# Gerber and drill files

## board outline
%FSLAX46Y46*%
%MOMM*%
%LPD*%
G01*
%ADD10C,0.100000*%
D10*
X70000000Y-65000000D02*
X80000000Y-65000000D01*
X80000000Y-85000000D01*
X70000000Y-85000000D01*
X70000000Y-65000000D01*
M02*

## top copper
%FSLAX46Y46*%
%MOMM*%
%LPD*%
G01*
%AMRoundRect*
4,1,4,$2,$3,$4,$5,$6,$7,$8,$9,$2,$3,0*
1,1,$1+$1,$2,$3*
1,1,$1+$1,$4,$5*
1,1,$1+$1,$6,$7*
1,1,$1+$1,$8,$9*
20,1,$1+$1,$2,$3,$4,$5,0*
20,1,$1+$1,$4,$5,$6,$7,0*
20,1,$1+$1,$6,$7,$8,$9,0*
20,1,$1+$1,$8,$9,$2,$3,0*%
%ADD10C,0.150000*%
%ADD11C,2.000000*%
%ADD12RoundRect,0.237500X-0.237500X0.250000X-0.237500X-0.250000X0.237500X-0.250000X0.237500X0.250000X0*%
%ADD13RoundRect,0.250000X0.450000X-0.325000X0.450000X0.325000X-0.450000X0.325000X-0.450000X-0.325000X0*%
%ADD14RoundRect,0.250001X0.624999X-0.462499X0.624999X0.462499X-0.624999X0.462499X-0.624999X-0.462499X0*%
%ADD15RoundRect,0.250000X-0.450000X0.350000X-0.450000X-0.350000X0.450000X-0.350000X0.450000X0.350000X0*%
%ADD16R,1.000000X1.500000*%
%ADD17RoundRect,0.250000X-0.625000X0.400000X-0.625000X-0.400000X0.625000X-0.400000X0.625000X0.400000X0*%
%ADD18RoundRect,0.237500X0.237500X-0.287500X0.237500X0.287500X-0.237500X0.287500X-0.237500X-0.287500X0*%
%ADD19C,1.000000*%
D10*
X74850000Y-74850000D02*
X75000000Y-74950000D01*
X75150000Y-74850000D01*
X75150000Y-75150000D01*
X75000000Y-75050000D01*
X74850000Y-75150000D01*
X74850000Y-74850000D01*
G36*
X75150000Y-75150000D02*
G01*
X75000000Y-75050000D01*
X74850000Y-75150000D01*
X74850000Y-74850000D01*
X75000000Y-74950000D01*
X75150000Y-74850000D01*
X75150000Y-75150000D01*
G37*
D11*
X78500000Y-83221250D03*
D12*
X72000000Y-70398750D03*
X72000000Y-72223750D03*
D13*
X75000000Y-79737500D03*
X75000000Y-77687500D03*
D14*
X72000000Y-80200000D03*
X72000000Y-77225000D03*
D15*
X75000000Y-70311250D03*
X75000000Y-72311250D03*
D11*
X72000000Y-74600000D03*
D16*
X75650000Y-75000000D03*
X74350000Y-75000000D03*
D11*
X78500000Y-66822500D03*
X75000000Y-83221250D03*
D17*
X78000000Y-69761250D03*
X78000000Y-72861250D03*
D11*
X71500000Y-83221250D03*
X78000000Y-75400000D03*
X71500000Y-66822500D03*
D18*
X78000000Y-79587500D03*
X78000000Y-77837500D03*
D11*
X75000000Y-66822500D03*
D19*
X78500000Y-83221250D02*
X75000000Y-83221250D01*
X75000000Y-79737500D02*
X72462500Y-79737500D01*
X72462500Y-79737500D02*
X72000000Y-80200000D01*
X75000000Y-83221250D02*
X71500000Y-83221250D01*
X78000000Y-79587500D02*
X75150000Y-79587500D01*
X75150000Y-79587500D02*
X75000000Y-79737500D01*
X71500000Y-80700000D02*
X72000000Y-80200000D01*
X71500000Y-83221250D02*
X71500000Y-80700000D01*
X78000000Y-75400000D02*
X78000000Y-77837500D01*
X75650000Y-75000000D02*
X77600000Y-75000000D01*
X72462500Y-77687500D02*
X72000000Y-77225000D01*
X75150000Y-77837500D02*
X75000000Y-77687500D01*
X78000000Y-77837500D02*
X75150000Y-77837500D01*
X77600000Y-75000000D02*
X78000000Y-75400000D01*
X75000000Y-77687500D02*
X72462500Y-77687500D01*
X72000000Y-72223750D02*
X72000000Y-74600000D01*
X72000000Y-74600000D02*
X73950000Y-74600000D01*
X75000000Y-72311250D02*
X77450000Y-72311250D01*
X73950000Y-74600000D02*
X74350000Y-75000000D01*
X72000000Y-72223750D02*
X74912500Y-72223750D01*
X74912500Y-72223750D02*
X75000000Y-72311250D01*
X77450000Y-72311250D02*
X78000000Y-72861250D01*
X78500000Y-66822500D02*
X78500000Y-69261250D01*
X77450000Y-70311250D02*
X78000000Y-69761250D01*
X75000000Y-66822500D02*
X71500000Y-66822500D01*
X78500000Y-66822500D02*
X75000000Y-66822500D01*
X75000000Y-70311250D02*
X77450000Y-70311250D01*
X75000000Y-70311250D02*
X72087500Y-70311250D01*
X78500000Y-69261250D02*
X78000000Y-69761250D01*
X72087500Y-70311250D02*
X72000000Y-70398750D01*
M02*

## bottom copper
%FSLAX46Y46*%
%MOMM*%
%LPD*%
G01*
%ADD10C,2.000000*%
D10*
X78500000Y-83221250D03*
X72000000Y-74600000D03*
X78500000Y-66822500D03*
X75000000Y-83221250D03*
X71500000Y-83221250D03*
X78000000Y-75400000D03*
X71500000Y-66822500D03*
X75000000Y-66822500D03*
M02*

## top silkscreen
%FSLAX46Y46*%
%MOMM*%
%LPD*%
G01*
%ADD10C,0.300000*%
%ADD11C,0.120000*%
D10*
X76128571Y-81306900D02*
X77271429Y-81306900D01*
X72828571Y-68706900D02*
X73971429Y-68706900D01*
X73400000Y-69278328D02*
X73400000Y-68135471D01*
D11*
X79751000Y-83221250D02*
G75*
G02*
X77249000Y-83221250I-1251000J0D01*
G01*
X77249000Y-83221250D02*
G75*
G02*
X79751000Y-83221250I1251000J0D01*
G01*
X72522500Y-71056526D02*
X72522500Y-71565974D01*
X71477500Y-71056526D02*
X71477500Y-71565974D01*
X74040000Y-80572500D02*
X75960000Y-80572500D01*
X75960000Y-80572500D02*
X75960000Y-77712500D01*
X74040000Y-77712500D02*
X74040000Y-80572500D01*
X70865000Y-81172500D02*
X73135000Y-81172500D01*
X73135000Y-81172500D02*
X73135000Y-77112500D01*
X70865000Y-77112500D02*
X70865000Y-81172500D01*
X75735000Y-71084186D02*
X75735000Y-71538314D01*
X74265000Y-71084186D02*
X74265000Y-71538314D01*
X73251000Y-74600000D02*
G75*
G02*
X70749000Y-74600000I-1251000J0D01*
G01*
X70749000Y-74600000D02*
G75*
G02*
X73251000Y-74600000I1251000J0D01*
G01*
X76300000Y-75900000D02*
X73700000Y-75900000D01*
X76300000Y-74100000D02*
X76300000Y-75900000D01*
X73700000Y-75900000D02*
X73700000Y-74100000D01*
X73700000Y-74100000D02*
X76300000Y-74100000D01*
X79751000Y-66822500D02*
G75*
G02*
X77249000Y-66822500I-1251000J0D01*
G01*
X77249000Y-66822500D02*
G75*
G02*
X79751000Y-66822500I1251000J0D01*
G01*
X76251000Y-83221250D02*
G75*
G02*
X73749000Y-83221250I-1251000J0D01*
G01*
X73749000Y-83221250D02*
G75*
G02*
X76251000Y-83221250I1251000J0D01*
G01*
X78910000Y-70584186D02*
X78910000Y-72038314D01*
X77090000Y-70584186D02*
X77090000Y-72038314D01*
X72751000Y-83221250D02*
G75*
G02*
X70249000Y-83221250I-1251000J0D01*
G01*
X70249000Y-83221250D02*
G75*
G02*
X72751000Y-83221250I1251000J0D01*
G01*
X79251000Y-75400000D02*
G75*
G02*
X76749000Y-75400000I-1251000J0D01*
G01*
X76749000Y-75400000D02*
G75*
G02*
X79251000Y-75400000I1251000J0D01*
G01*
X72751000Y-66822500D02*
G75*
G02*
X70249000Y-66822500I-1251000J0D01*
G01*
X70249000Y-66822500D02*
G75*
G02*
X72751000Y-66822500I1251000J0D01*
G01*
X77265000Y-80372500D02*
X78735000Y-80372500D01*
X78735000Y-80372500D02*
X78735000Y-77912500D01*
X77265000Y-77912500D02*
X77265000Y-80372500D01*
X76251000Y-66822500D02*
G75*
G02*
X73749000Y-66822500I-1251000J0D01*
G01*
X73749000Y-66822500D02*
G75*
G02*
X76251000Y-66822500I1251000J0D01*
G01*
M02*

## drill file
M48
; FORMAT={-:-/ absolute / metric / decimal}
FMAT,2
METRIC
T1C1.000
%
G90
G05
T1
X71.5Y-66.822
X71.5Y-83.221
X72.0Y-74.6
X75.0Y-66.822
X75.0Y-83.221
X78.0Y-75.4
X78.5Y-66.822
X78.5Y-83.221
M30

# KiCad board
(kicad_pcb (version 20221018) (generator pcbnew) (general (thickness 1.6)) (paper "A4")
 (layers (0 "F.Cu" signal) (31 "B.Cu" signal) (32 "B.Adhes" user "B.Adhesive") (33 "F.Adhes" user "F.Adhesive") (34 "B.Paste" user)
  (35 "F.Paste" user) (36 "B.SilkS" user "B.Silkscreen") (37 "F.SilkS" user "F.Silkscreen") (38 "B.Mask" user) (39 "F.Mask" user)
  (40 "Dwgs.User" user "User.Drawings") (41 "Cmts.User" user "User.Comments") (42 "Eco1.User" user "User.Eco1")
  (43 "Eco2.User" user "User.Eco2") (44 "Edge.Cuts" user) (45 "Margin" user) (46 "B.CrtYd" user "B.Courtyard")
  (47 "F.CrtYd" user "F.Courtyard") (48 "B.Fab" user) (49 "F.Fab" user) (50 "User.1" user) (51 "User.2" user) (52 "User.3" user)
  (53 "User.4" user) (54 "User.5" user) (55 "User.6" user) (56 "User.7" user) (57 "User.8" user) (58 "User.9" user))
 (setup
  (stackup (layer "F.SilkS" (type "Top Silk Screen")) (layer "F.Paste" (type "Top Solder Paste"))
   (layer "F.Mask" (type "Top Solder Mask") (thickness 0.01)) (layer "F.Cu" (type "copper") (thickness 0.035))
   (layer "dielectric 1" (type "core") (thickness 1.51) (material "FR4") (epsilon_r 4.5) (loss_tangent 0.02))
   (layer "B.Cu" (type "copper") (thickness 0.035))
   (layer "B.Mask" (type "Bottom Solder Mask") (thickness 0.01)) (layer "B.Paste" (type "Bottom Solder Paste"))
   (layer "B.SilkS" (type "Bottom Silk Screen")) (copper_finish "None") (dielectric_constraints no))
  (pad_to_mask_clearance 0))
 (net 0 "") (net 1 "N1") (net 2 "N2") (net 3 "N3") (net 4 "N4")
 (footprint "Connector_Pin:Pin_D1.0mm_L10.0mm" (layer "F.Cu") (at 78.5 83.22125)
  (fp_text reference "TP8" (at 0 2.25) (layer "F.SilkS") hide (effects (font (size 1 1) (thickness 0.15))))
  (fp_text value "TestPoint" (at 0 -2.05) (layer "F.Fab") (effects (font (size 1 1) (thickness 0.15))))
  (fp_circle (center 0 0) (end 1.25 0.05) (stroke (width 0.12) (type solid)) (fill none) (layer "F.SilkS"))
  (pad "1" thru_hole circle (at 0 0) (size 2 2) (drill 1) (layers "*.Cu" "*.Mask") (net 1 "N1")))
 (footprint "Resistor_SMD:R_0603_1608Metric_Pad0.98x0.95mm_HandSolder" (layer "F.Cu") (at 72 71.31125 -90)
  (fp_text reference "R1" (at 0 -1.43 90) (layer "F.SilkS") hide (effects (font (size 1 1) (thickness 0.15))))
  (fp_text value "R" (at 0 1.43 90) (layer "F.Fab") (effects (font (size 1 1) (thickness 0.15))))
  (fp_line (start -0.254724 -0.5225) (end 0.254724 -0.5225) (stroke (width 0.12) (type solid)) (layer "F.SilkS"))
  (fp_line (start -0.254724 0.5225) (end 0.254724 0.5225) (stroke (width 0.12) (type solid)) (layer "F.SilkS"))
  (pad "1" smd roundrect (at -0.9125 0 270) (size 0.975 0.95) (layers "F.Cu" "F.Paste" "F.Mask") (roundrect_rratio 0.25) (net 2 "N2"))
  (pad "2" smd roundrect (at 0.9125 0 270) (size 0.975 0.95) (layers "F.Cu" "F.Paste" "F.Mask") (roundrect_rratio 0.25) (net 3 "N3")))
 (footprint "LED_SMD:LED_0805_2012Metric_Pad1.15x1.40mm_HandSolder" (layer "F.Cu") (at 75 78.7125 90)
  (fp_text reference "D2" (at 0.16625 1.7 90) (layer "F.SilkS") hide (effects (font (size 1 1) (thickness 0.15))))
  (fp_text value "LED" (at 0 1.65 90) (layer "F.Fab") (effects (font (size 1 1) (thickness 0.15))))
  (fp_line (start -1.86 -0.96) (end -1.86 0.96) (stroke (width 0.12) (type solid)) (layer "F.SilkS"))
  (fp_line (start -1.86 0.96) (end 1 0.96) (stroke (width 0.12) (type solid)) (layer "F.SilkS"))
  (fp_line (start 1 -0.96) (end -1.86 -0.96) (stroke (width 0.12) (type solid)) (layer "F.SilkS"))
  (pad "1" smd roundrect (at -1.025 0 90) (size 1.15 1.4) (layers "F.Cu" "F.Paste" "F.Mask") (roundrect_rratio 0.2173913043) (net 1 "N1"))
  (pad "2" smd roundrect (at 1.025 0 90) (size 1.15 1.4) (layers "F.Cu" "F.Paste" "F.Mask") (roundrect_rratio 0.2173913043) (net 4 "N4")))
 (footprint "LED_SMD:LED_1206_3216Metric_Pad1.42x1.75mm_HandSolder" (layer "F.Cu") (at 72 78.7125 90)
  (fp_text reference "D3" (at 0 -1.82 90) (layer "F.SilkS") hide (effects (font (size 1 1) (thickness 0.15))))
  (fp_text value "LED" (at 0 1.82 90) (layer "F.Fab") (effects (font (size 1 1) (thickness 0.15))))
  (fp_line (start -2.46 -1.135) (end -2.46 1.135) (stroke (width 0.12) (type solid)) (layer "F.SilkS"))
  (fp_line (start -2.46 1.135) (end 1.6 1.135) (stroke (width 0.12) (type solid)) (layer "F.SilkS"))
  (fp_line (start 1.6 -1.135) (end -2.46 -1.135) (stroke (width 0.12) (type solid)) (layer "F.SilkS"))
  (pad "1" smd roundrect (at -1.4875 0 90) (size 1.425 1.75) (layers "F.Cu" "F.Paste" "F.Mask") (roundrect_rratio 0.1754392982) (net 1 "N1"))
  (pad "2" smd roundrect (at 1.4875 0 90) (size 1.425 1.75) (layers "F.Cu" "F.Paste" "F.Mask") (roundrect_rratio 0.1754392982) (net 4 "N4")))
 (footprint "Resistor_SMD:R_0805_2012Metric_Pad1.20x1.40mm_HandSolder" (layer "F.Cu") (at 75 71.31125 -90)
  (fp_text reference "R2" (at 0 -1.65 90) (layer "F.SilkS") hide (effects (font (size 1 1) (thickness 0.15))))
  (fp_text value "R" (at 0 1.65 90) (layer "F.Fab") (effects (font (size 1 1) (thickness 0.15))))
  (fp_line (start -0.227064 -0.735) (end 0.227064 -0.735) (stroke (width 0.12) (type solid)) (layer "F.SilkS"))
  (fp_line (start -0.227064 0.735) (end 0.227064 0.735) (stroke (width 0.12) (type solid)) (layer "F.SilkS"))
  (pad "1" smd roundrect (at -1 0 270) (size 1.2 1.4) (layers "F.Cu" "F.Paste" "F.Mask") (roundrect_rratio 0.2083333333) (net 2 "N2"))
  (pad "2" smd roundrect (at 1 0 270) (size 1.2 1.4) (layers "F.Cu" "F.Paste" "F.Mask") (roundrect_rratio 0.2083333333) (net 3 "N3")))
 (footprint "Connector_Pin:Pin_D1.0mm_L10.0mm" (layer "F.Cu") (at 72 74.6)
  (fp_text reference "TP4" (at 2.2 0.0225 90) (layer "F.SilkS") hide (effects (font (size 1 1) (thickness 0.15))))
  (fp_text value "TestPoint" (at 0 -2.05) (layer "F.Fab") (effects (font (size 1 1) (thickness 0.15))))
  (fp_circle (center 0 0) (end 1.25 0.05) (stroke (width 0.12) (type solid)) (fill none) (layer "F.SilkS"))
  (pad "1" thru_hole circle (at 0 0) (size 2 2) (drill 1) (layers "*.Cu" "*.Mask") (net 3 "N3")))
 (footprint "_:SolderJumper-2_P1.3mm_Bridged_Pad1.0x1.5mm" (layer "F.Cu") (at 75 75 180) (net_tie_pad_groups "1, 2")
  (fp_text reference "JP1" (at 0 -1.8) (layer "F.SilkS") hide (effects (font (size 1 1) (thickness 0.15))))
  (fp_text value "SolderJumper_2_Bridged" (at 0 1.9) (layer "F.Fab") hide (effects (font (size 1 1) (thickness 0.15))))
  (fp_poly
   (pts (xy 0.15 0.15) (xy 0 0.05) (xy -0.15 0.15) (xy -0.15 -0.15) (xy 0 -0.05) (xy 0.15 -0.15)) (stroke (width 0.15) (type solid))
   (fill solid) (layer "F.Cu"))
  (fp_line (start -1.3 -0.9) (end 1.3 -0.9) (stroke (width 0.12) (type solid)) (layer "F.SilkS"))
  (fp_line (start -1.3 0.9) (end -1.3 -0.9) (stroke (width 0.12) (type solid)) (layer "F.SilkS"))
  (fp_line (start 1.3 -0.9) (end 1.3 0.9) (stroke (width 0.12) (type solid)) (layer "F.SilkS"))
  (fp_line (start 1.3 0.9) (end -1.3 0.9) (stroke (width 0.12) (type solid)) (layer "F.SilkS"))
  (pad "1" smd rect (at -0.65 0 180) (size 1 1.5) (layers "F.Cu" "F.Mask") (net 4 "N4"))
  (pad "2" smd rect (at 0.65 0 180) (size 1 1.5) (layers "F.Cu" "F.Mask") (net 3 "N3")))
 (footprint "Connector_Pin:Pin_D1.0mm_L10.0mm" (layer "F.Cu") (at 78.5 66.8225)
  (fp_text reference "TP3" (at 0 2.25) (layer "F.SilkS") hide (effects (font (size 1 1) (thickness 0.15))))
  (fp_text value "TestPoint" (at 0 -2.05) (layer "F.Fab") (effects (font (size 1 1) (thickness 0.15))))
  (fp_circle (center 0 0) (end 1.25 0.05) (stroke (width 0.12) (type solid)) (fill none) (layer "F.SilkS"))
  (pad "1" thru_hole circle (at 0 0) (size 2 2) (drill 1) (layers "*.Cu" "*.Mask") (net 2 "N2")))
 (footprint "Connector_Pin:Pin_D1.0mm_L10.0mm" (layer "F.Cu") (at 75 83.22125)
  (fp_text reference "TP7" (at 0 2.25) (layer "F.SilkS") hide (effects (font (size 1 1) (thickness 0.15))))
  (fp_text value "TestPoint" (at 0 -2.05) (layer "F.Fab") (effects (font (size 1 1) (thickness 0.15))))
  (fp_circle (center 0 0) (end 1.25 0.05) (stroke (width 0.12) (type solid)) (fill none) (layer "F.SilkS"))
  (pad "1" thru_hole circle (at 0 0) (size 2 2) (drill 1) (layers "*.Cu" "*.Mask") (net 1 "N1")))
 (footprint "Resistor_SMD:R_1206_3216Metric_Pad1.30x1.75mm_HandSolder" (layer "F.Cu") (at 78 71.31125 -90)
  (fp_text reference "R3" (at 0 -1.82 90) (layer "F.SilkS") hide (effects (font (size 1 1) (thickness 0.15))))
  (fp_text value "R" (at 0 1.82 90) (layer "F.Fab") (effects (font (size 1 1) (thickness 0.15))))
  (fp_line (start -0.727064 -0.91) (end 0.727064 -0.91) (stroke (width 0.12) (type solid)) (layer "F.SilkS"))
  (fp_line (start -0.727064 0.91) (end 0.727064 0.91) (stroke (width 0.12) (type solid)) (layer "F.SilkS"))
  (pad "1" smd roundrect (at -1.55 0 270) (size 1.3 1.75) (layers "F.Cu" "F.Paste" "F.Mask") (roundrect_rratio 0.1923076923) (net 2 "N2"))
  (pad "2" smd roundrect (at 1.55 0 270) (size 1.3 1.75) (layers "F.Cu" "F.Paste" "F.Mask") (roundrect_rratio 0.1923076923) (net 3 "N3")))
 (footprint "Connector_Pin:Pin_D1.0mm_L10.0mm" (layer "F.Cu") (at 71.5 83.22125)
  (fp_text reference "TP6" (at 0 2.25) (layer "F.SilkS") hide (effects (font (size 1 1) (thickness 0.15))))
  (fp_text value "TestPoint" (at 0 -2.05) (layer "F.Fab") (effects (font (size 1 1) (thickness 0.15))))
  (fp_circle (center 0 0) (end 1.25 0.05) (stroke (width 0.12) (type solid)) (fill none) (layer "F.SilkS"))
  (pad "1" thru_hole circle (at 0 0) (size 2 2) (drill 1) (layers "*.Cu" "*.Mask") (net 1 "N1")))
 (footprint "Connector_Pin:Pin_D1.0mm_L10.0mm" (layer "F.Cu") (at 78 75.4)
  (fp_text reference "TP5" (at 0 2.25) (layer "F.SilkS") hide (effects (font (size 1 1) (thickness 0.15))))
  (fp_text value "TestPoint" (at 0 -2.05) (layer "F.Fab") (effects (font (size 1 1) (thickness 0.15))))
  (fp_circle (center 0 0) (end 1.25 0.05) (stroke (width 0.12) (type solid)) (fill none) (layer "F.SilkS"))
  (pad "1" thru_hole circle (at 0 0) (size 2 2) (drill 1) (layers "*.Cu" "*.Mask") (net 4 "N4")))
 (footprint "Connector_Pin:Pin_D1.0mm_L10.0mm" (layer "F.Cu") (at 71.5 66.8225)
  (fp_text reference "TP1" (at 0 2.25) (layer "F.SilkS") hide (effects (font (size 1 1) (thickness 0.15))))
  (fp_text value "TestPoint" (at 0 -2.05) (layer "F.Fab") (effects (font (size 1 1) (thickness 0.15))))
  (fp_circle (center 0 0) (end 1.25 0.05) (stroke (width 0.12) (type solid)) (fill none) (layer "F.SilkS"))
  (pad "1" thru_hole circle (at 0 0) (size 2 2) (drill 1) (layers "*.Cu" "*.Mask") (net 2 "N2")))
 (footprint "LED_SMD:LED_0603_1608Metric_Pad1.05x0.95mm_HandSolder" (layer "F.Cu") (at 78 78.7125 90)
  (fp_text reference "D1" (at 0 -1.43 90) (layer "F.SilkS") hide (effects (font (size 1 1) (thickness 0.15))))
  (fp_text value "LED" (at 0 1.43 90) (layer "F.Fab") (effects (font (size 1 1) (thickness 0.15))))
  (fp_line (start -1.66 -0.735) (end -1.66 0.735) (stroke (width 0.12) (type solid)) (layer "F.SilkS"))
  (fp_line (start -1.66 0.735) (end 0.8 0.735) (stroke (width 0.12) (type solid)) (layer "F.SilkS"))
  (fp_line (start 0.8 -0.735) (end -1.66 -0.735) (stroke (width 0.12) (type solid)) (layer "F.SilkS"))
  (pad "1" smd roundrect (at -0.875 0 90) (size 1.05 0.95) (layers "F.Cu" "F.Paste" "F.Mask") (roundrect_rratio 0.25) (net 1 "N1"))
  (pad "2" smd roundrect (at 0.875 0 90) (size 1.05 0.95) (layers "F.Cu" "F.Paste" "F.Mask") (roundrect_rratio 0.25) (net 4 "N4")))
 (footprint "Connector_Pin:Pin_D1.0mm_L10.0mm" (layer "F.Cu") (at 75 66.8225)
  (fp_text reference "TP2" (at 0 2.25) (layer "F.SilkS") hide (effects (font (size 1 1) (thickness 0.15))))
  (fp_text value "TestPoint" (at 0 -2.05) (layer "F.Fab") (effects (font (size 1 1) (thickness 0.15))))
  (fp_circle (center 0 0) (end 1.25 0.05) (stroke (width 0.12) (type solid)) (fill none) (layer "F.SilkS"))
  (pad "1" thru_hole circle (at 0 0) (size 2 2) (drill 1) (layers "*.Cu" "*.Mask") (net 2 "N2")))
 (gr_rect (start 70 65) (end 80 85) (stroke (width 0.1) (type solid)) (fill none) (layer "Edge.Cuts"))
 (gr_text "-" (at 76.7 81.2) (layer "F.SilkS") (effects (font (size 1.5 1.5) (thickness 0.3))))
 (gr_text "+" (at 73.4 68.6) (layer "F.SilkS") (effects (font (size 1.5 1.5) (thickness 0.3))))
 (segment (start 78.5 83.22125) (end 75 83.22125) (width 1) (layer "F.Cu") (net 1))
 (segment (start 75 79.7375) (end 72.4625 79.7375) (width 1) (layer "F.Cu") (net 1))
 (segment (start 72.4625 79.7375) (end 72 80.2) (width 1) (layer "F.Cu") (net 1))
 (segment (start 75 83.22125) (end 71.5 83.22125) (width 1) (layer "F.Cu") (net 1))
 (segment (start 78 79.5875) (end 75.15 79.5875) (width 1) (layer "F.Cu") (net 1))
 (segment (start 75.15 79.5875) (end 75 79.7375) (width 1) (layer "F.Cu") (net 1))
 (segment (start 71.5 80.7) (end 72 80.2) (width 1) (layer "F.Cu") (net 1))
 (segment (start 71.5 83.22125) (end 71.5 80.7) (width 1) (layer "F.Cu") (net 1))
 (segment (start 78 75.4) (end 78 77.8375) (width 1) (layer "F.Cu") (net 4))
 (segment (start 75.65 75) (end 77.6 75) (width 1) (layer "F.Cu") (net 4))
 (segment (start 72.4625 77.6875) (end 72 77.225) (width 1) (layer "F.Cu") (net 4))
 (segment (start 75.15 77.8375) (end 75 77.6875) (width 1) (layer "F.Cu") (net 4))
 (segment (start 78 77.8375) (end 75.15 77.8375) (width 1) (layer "F.Cu") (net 4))
 (segment (start 77.6 75) (end 78 75.4) (width 1) (layer "F.Cu") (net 4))
 (segment (start 75 77.6875) (end 72.4625 77.6875) (width 1) (layer "F.Cu") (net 4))
 (segment (start 72 72.22375) (end 72 74.6) (width 1) (layer "F.Cu") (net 3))
 (segment (start 72 74.6) (end 73.95 74.6) (width 1) (layer "F.Cu") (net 3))
 (segment (start 75 72.31125) (end 77.45 72.31125) (width 1) (layer "F.Cu") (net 3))
 (segment (start 73.95 74.6) (end 74.35 75) (width 1) (layer "F.Cu") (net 3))
 (segment (start 72 72.22375) (end 74.9125 72.22375) (width 1) (layer "F.Cu") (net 3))
 (segment (start 74.9125 72.22375) (end 75 72.31125) (width 1) (layer "F.Cu") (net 3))
 (segment (start 77.45 72.31125) (end 78 72.86125) (width 1) (layer "F.Cu") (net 3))
 (segment (start 78.5 66.8225) (end 78.5 69.26125) (width 1) (layer "F.Cu") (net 2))
 (segment (start 77.45 70.31125) (end 78 69.76125) (width 1) (layer "F.Cu") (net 2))
 (segment (start 75 66.8225) (end 71.5 66.8225) (width 1) (layer "F.Cu") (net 2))
 (segment (start 78.5 66.8225) (end 75 66.8225) (width 1) (layer "F.Cu") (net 2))
 (segment (start 75 70.31125) (end 77.45 70.31125) (width 1) (layer "F.Cu") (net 2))
 (segment (start 75 70.31125) (end 72.0875 70.31125) (width 1) (layer "F.Cu") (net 2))
 (segment (start 78.5 69.26125) (end 78 69.76125) (width 1) (layer "F.Cu") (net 2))
 (segment (start 72.0875 70.31125) (end 72 70.39875) (width 1) (layer "F.Cu") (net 2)))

